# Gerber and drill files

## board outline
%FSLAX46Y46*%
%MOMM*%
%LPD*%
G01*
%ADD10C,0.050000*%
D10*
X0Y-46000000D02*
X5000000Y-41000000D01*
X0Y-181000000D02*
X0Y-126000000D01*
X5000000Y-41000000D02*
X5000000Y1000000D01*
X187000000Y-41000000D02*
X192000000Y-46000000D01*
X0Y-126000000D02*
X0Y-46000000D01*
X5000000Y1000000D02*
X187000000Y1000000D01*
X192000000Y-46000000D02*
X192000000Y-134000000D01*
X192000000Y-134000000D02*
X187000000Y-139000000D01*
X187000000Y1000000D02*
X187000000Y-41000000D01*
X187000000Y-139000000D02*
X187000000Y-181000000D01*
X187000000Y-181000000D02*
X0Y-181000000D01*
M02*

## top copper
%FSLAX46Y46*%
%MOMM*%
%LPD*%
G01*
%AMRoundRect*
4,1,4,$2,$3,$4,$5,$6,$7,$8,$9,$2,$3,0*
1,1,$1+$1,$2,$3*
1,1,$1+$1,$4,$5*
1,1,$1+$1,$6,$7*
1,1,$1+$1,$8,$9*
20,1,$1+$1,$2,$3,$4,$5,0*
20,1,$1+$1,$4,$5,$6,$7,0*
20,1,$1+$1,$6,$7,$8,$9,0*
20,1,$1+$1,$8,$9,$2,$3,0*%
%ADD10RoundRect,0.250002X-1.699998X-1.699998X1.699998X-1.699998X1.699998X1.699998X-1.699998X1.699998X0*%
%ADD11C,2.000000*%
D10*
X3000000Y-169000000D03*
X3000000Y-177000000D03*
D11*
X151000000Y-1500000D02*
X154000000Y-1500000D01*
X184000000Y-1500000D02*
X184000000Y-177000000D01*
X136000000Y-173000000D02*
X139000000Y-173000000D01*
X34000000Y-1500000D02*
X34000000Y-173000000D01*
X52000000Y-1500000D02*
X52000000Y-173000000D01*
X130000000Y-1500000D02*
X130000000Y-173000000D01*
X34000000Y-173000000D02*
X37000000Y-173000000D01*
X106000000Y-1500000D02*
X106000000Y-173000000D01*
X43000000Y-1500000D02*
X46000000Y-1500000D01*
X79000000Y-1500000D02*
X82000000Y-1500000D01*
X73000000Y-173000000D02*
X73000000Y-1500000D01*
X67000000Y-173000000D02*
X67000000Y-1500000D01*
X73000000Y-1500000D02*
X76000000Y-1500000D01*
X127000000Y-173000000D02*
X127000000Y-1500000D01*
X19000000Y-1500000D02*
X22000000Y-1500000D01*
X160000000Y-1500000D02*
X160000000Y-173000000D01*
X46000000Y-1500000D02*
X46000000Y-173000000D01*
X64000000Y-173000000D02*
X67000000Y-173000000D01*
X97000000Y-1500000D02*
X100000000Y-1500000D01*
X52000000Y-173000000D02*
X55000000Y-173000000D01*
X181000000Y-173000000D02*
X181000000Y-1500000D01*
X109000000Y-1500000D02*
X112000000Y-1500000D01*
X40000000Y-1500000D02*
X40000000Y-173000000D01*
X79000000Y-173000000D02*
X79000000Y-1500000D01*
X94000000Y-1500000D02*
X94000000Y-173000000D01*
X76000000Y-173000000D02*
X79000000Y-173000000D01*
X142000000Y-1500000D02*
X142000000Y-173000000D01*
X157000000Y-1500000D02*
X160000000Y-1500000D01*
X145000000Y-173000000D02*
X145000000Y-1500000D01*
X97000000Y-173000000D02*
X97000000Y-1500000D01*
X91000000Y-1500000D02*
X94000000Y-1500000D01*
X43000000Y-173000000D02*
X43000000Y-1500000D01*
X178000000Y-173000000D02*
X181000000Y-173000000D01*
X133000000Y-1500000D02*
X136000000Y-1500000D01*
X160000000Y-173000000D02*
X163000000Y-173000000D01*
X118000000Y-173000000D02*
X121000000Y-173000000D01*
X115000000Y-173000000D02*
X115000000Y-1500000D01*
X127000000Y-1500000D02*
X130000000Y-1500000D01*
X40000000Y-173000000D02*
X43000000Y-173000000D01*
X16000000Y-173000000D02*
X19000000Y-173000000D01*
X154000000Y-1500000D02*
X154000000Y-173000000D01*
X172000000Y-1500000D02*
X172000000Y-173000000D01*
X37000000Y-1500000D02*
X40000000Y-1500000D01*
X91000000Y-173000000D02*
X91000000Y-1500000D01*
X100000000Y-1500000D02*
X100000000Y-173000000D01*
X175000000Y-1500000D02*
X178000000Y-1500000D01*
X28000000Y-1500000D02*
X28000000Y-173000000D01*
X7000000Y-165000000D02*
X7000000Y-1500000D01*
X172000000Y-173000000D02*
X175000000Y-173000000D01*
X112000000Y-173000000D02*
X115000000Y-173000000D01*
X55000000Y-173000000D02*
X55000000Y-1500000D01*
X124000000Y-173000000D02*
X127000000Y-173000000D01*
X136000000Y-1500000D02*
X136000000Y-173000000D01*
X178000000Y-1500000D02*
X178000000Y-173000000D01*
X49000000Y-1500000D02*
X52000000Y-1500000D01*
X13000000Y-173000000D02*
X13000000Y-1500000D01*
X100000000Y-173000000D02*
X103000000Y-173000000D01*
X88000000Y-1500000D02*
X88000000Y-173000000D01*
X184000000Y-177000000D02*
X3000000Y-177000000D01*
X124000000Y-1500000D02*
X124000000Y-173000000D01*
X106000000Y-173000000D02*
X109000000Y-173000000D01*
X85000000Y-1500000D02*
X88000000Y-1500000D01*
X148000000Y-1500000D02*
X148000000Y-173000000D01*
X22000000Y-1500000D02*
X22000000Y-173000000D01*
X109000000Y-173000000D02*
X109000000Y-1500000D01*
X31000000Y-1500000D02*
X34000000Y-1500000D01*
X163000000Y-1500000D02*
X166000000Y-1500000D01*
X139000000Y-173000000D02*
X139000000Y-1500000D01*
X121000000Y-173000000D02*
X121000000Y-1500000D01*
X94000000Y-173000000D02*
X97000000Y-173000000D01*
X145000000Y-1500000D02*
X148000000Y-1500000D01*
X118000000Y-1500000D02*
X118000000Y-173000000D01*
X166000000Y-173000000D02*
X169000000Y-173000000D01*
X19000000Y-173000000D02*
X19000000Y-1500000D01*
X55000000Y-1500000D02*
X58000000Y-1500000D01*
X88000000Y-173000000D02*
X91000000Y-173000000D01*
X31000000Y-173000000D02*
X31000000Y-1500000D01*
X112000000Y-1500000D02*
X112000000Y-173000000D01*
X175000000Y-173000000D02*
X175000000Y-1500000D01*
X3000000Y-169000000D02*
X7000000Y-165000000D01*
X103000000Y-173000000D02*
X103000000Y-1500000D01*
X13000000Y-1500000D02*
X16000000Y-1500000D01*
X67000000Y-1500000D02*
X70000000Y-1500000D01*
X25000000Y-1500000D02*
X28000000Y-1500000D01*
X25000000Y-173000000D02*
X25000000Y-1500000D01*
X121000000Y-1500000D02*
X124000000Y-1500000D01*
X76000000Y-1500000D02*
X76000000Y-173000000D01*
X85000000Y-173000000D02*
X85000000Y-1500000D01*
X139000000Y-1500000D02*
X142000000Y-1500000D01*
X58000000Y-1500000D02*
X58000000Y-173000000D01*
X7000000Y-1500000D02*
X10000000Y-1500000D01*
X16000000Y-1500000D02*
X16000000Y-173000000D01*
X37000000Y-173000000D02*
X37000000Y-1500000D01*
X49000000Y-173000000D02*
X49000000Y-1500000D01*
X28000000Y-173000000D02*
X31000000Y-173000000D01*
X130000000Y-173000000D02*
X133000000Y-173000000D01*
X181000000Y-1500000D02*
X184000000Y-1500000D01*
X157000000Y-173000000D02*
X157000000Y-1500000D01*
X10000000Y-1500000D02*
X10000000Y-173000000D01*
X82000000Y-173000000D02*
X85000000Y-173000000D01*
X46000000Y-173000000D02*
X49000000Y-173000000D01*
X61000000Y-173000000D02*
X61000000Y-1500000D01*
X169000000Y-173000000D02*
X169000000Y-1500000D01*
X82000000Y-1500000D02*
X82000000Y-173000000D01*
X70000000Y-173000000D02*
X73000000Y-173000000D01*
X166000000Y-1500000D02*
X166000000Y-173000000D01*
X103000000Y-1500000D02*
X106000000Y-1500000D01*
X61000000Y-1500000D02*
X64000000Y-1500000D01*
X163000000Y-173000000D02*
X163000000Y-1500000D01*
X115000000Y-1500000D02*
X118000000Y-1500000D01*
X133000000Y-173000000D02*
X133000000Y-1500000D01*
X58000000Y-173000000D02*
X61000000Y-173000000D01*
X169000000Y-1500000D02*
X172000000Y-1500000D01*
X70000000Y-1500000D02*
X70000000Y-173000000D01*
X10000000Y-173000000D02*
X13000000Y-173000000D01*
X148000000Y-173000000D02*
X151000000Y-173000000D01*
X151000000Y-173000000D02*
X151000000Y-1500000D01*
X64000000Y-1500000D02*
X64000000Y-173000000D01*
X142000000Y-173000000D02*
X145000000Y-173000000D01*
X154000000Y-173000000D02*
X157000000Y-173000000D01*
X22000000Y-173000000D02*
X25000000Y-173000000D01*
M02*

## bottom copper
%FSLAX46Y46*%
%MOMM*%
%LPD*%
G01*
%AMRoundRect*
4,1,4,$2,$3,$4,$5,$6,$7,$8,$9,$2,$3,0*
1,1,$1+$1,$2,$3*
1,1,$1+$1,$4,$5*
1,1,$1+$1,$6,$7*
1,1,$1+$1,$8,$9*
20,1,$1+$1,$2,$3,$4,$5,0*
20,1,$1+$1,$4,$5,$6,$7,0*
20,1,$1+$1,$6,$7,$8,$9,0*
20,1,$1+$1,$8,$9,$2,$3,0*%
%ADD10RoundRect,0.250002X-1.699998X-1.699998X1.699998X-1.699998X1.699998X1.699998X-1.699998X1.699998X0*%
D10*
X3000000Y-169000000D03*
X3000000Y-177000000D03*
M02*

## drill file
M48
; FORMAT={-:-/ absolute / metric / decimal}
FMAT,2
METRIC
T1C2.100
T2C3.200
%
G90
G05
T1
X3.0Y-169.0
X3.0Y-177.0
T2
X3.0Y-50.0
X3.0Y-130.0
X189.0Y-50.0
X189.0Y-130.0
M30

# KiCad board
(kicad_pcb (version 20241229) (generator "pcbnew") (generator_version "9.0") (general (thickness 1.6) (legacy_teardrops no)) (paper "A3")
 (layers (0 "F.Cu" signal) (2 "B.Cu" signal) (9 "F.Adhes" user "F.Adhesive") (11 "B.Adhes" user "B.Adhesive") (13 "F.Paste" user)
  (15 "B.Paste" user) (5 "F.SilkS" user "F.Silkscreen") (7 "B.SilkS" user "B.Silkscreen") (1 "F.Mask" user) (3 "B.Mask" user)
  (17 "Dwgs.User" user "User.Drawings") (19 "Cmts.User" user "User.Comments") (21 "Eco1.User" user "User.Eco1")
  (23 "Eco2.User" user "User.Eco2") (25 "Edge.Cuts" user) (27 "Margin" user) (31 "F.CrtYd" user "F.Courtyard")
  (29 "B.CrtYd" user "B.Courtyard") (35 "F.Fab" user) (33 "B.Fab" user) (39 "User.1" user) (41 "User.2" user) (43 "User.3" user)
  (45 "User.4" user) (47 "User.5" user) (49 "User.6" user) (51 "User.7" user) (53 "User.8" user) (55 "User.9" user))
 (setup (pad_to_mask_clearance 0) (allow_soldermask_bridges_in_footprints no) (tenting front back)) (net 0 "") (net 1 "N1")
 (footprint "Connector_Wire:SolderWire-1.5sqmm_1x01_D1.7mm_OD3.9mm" (layer "F.Cu") (at 3 169)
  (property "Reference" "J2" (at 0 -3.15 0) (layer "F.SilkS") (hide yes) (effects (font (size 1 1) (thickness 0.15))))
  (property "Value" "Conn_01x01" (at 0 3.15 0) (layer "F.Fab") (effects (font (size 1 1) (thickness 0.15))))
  (pad "1" thru_hole roundrect (at 0 0) (size 3.9 3.9) (drill 2.1) (layers "*.Cu" "*.Mask") (remove_unused_layers no)
   (roundrect_rratio 0.064103) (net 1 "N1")))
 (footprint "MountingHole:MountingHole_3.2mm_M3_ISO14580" (layer "F.Cu") (at 189 50)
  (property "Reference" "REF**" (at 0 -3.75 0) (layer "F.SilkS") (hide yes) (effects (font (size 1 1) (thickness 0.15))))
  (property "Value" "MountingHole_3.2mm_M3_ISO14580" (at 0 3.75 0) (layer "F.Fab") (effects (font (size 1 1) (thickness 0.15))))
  (pad "" np_thru_hole circle (at 0 0) (size 3.2 3.2) (drill 3.2) (layers "*.Cu" "*.Mask")))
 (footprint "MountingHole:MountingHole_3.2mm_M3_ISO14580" (layer "F.Cu") (at 3 130)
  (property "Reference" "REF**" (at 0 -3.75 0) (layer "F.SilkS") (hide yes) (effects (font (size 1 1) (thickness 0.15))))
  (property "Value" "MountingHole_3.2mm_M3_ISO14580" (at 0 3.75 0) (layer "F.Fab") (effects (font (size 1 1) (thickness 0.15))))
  (pad "" np_thru_hole circle (at 0 0) (size 3.2 3.2) (drill 3.2) (layers "*.Cu" "*.Mask")))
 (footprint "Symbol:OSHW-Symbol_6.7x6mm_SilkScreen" (layer "F.Cu") (at 12 175)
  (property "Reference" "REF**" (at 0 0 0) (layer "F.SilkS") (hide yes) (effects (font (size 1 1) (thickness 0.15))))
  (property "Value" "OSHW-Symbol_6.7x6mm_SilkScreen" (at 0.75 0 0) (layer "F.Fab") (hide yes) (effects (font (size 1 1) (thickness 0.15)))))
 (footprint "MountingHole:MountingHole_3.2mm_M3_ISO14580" (layer "F.Cu") (at 189 130)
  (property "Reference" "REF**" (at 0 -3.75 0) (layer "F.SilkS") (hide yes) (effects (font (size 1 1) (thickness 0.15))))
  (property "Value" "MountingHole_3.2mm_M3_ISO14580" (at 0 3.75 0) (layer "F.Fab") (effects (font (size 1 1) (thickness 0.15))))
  (pad "" np_thru_hole circle (at 0 0) (size 3.2 3.2) (drill 3.2) (layers "*.Cu" "*.Mask")))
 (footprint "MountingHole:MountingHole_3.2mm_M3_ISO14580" (layer "F.Cu") (at 3 50)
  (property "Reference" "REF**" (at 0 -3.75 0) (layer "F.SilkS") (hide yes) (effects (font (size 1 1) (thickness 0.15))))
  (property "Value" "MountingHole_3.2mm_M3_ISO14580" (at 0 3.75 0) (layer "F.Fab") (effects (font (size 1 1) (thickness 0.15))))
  (pad "" np_thru_hole circle (at 0 0) (size 3.2 3.2) (drill 3.2) (layers "*.Cu" "*.Mask")))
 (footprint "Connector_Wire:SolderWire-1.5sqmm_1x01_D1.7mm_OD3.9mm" (layer "F.Cu") (at 3 177)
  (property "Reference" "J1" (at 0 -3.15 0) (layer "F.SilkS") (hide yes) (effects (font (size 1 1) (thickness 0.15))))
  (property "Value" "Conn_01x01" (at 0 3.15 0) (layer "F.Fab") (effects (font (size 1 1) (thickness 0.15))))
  (pad "1" thru_hole roundrect (at 0 0) (size 3.9 3.9) (drill 2.1) (layers "*.Cu" "*.Mask") (remove_unused_layers no)
   (roundrect_rratio 0.064103) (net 1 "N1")))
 (gr_line (start 0 46) (end 5 41) (stroke (width 0.05) (type default)) (layer "Edge.Cuts"))
 (gr_line (start 0 181) (end 0 126) (stroke (width 0.05) (type default)) (layer "Edge.Cuts"))
 (gr_line (start 5 41) (end 5 -1) (stroke (width 0.05) (type default)) (layer "Edge.Cuts"))
 (gr_line (start 187 41) (end 192 46) (stroke (width 0.05) (type default)) (layer "Edge.Cuts"))
 (gr_line (start 0 126) (end 0 46) (stroke (width 0.05) (type default)) (layer "Edge.Cuts"))
 (gr_line (start 5 -1) (end 187 -1) (stroke (width 0.05) (type default)) (layer "Edge.Cuts"))
 (gr_line (start 192 46) (end 192 134) (stroke (width 0.05) (type default)) (layer "Edge.Cuts"))
 (gr_line (start 192 134) (end 187 139) (stroke (width 0.05) (type default)) (layer "Edge.Cuts"))
 (gr_line (start 187 -1) (end 187 41) (stroke (width 0.05) (type default)) (layer "Edge.Cuts"))
 (gr_line (start 187 139) (end 187 181) (stroke (width 0.05) (type default)) (layer "Edge.Cuts"))
 (gr_line (start 187 181) (end 0 181) (stroke (width 0.05) (type default)) (layer "Edge.Cuts"))
 (segment (start 151 1.5) (end 154 1.5) (width 2) (layer "F.Cu") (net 1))
 (segment (start 184 1.5) (end 184 177) (width 2) (layer "F.Cu") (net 1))
 (segment (start 136 173) (end 139 173) (width 2) (layer "F.Cu") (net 1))
 (segment (start 34 1.5) (end 34 173) (width 2) (layer "F.Cu") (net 1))
 (segment (start 52 1.5) (end 52 173) (width 2) (layer "F.Cu") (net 1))
 (segment (start 130 1.5) (end 130 173) (width 2) (layer "F.Cu") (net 1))
 (segment (start 34 173) (end 37 173) (width 2) (layer "F.Cu") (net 1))
 (segment (start 106 1.5) (end 106 173) (width 2) (layer "F.Cu") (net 1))
 (segment (start 43 1.5) (end 46 1.5) (width 2) (layer "F.Cu") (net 1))
 (segment (start 79 1.5) (end 82 1.5) (width 2) (layer "F.Cu") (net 1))
 (segment (start 73 173) (end 73 1.5) (width 2) (layer "F.Cu") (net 1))
 (segment (start 67 173) (end 67 1.5) (width 2) (layer "F.Cu") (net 1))
 (segment (start 73 1.5) (end 76 1.5) (width 2) (layer "F.Cu") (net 1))
 (segment (start 127 173) (end 127 1.5) (width 2) (layer "F.Cu") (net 1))
 (segment (start 19 1.5) (end 22 1.5) (width 2) (layer "F.Cu") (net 1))
 (segment (start 160 1.5) (end 160 173) (width 2) (layer "F.Cu") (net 1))
 (segment (start 46 1.5) (end 46 173) (width 2) (layer "F.Cu") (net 1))
 (segment (start 64 173) (end 67 173) (width 2) (layer "F.Cu") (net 1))
 (segment (start 97 1.5) (end 100 1.5) (width 2) (layer "F.Cu") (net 1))
 (segment (start 52 173) (end 55 173) (width 2) (layer "F.Cu") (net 1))
 (segment (start 181 173) (end 181 1.5) (width 2) (layer "F.Cu") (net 1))
 (segment (start 109 1.5) (end 112 1.5) (width 2) (layer "F.Cu") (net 1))
 (segment (start 40 1.5) (end 40 173) (width 2) (layer "F.Cu") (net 1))
 (segment (start 79 173) (end 79 1.5) (width 2) (layer "F.Cu") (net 1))
 (segment (start 94 1.5) (end 94 173) (width 2) (layer "F.Cu") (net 1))
 (segment (start 76 173) (end 79 173) (width 2) (layer "F.Cu") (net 1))
 (segment (start 142 1.5) (end 142 173) (width 2) (layer "F.Cu") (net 1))
 (segment (start 157 1.5) (end 160 1.5) (width 2) (layer "F.Cu") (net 1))
 (segment (start 145 173) (end 145 1.5) (width 2) (layer "F.Cu") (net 1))
 (segment (start 97 173) (end 97 1.5) (width 2) (layer "F.Cu") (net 1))
 (segment (start 91 1.5) (end 94 1.5) (width 2) (layer "F.Cu") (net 1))
 (segment (start 43 173) (end 43 1.5) (width 2) (layer "F.Cu") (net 1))
 (segment (start 178 173) (end 181 173) (width 2) (layer "F.Cu") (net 1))
 (segment (start 133 1.5) (end 136 1.5) (width 2) (layer "F.Cu") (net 1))
 (segment (start 160 173) (end 163 173) (width 2) (layer "F.Cu") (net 1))
 (segment (start 118 173) (end 121 173) (width 2) (layer "F.Cu") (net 1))
 (segment (start 115 173) (end 115 1.5) (width 2) (layer "F.Cu") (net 1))
 (segment (start 127 1.5) (end 130 1.5) (width 2) (layer "F.Cu") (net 1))
 (segment (start 40 173) (end 43 173) (width 2) (layer "F.Cu") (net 1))
 (segment (start 16 173) (end 19 173) (width 2) (layer "F.Cu") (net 1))
 (segment (start 154 1.5) (end 154 173) (width 2) (layer "F.Cu") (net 1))
 (segment (start 172 1.5) (end 172 173) (width 2) (layer "F.Cu") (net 1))
 (segment (start 37 1.5) (end 40 1.5) (width 2) (layer "F.Cu") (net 1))
 (segment (start 91 173) (end 91 1.5) (width 2) (layer "F.Cu") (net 1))
 (segment (start 100 1.5) (end 100 173) (width 2) (layer "F.Cu") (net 1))
 (segment (start 175 1.5) (end 178 1.5) (width 2) (layer "F.Cu") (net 1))
 (segment (start 28 1.5) (end 28 173) (width 2) (layer "F.Cu") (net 1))
 (segment (start 7 165) (end 7 1.5) (width 2) (layer "F.Cu") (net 1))
 (segment (start 172 173) (end 175 173) (width 2) (layer "F.Cu") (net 1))
 (segment (start 112 173) (end 115 173) (width 2) (layer "F.Cu") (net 1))
 (segment (start 55 173) (end 55 1.5) (width 2) (layer "F.Cu") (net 1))
 (segment (start 124 173) (end 127 173) (width 2) (layer "F.Cu") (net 1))
 (segment (start 136 1.5) (end 136 173) (width 2) (layer "F.Cu") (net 1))
 (segment (start 178 1.5) (end 178 173) (width 2) (layer "F.Cu") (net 1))
 (segment (start 49 1.5) (end 52 1.5) (width 2) (layer "F.Cu") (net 1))
 (segment (start 13 173) (end 13 1.5) (width 2) (layer "F.Cu") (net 1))
 (segment (start 100 173) (end 103 173) (width 2) (layer "F.Cu") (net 1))
 (segment (start 88 1.5) (end 88 173) (width 2) (layer "F.Cu") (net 1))
 (segment (start 184 177) (end 3 177) (width 2) (layer "F.Cu") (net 1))
 (segment (start 124 1.5) (end 124 173) (width 2) (layer "F.Cu") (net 1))
 (segment (start 106 173) (end 109 173) (width 2) (layer "F.Cu") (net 1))
 (segment (start 85 1.5) (end 88 1.5) (width 2) (layer "F.Cu") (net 1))
 (segment (start 148 1.5) (end 148 173) (width 2) (layer "F.Cu") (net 1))
 (segment (start 22 1.5) (end 22 173) (width 2) (layer "F.Cu") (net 1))
 (segment (start 109 173) (end 109 1.5) (width 2) (layer "F.Cu") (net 1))
 (segment (start 31 1.5) (end 34 1.5) (width 2) (layer "F.Cu") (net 1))
 (segment (start 163 1.5) (end 166 1.5) (width 2) (layer "F.Cu") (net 1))
 (segment (start 139 173) (end 139 1.5) (width 2) (layer "F.Cu") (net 1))
 (segment (start 121 173) (end 121 1.5) (width 2) (layer "F.Cu") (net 1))
 (segment (start 94 173) (end 97 173) (width 2) (layer "F.Cu") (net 1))
 (segment (start 145 1.5) (end 148 1.5) (width 2) (layer "F.Cu") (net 1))
 (segment (start 118 1.5) (end 118 173) (width 2) (layer "F.Cu") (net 1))
 (segment (start 166 173) (end 169 173) (width 2) (layer "F.Cu") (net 1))
 (segment (start 19 173) (end 19 1.5) (width 2) (layer "F.Cu") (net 1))
 (segment (start 55 1.5) (end 58 1.5) (width 2) (layer "F.Cu") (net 1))
 (segment (start 88 173) (end 91 173) (width 2) (layer "F.Cu") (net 1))
 (segment (start 31 173) (end 31 1.5) (width 2) (layer "F.Cu") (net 1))
 (segment (start 112 1.5) (end 112 173) (width 2) (layer "F.Cu") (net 1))
 (segment (start 175 173) (end 175 1.5) (width 2) (layer "F.Cu") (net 1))
 (segment (start 3 169) (end 7 165) (width 2) (layer "F.Cu") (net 1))
 (segment (start 103 173) (end 103 1.5) (width 2) (layer "F.Cu") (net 1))
 (segment (start 13 1.5) (end 16 1.5) (width 2) (layer "F.Cu") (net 1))
 (segment (start 67 1.5) (end 70 1.5) (width 2) (layer "F.Cu") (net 1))
 (segment (start 25 1.5) (end 28 1.5) (width 2) (layer "F.Cu") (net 1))
 (segment (start 25 173) (end 25 1.5) (width 2) (layer "F.Cu") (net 1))
 (segment (start 121 1.5) (end 124 1.5) (width 2) (layer "F.Cu") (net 1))
 (segment (start 76 1.5) (end 76 173) (width 2) (layer "F.Cu") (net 1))
 (segment (start 85 173) (end 85 1.5) (width 2) (layer "F.Cu") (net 1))
 (segment (start 139 1.5) (end 142 1.5) (width 2) (layer "F.Cu") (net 1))
 (segment (start 58 1.5) (end 58 173) (width 2) (layer "F.Cu") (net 1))
 (segment (start 7 1.5) (end 10 1.5) (width 2) (layer "F.Cu") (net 1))
 (segment (start 16 1.5) (end 16 173) (width 2) (layer "F.Cu") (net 1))
 (segment (start 37 173) (end 37 1.5) (width 2) (layer "F.Cu") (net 1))
 (segment (start 49 173) (end 49 1.5) (width 2) (layer "F.Cu") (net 1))
 (segment (start 28 173) (end 31 173) (width 2) (layer "F.Cu") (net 1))
 (segment (start 130 173) (end 133 173) (width 2) (layer "F.Cu") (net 1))
 (segment (start 181 1.5) (end 184 1.5) (width 2) (layer "F.Cu") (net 1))
 (segment (start 157 173) (end 157 1.5) (width 2) (layer "F.Cu") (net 1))
 (segment (start 10 1.5) (end 10 173) (width 2) (layer "F.Cu") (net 1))
 (segment (start 82 173) (end 85 173) (width 2) (layer "F.Cu") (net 1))
 (segment (start 46 173) (end 49 173) (width 2) (layer "F.Cu") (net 1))
 (segment (start 61 173) (end 61 1.5) (width 2) (layer "F.Cu") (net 1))
 (segment (start 169 173) (end 169 1.5) (width 2) (layer "F.Cu") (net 1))
 (segment (start 82 1.5) (end 82 173) (width 2) (layer "F.Cu") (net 1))
 (segment (start 70 173) (end 73 173) (width 2) (layer "F.Cu") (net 1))
 (segment (start 166 1.5) (end 166 173) (width 2) (layer "F.Cu") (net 1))
 (segment (start 103 1.5) (end 106 1.5) (width 2) (layer "F.Cu") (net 1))
 (segment (start 61 1.5) (end 64 1.5) (width 2) (layer "F.Cu") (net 1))
 (segment (start 163 173) (end 163 1.5) (width 2) (layer "F.Cu") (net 1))
 (segment (start 115 1.5) (end 118 1.5) (width 2) (layer "F.Cu") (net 1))
 (segment (start 133 173) (end 133 1.5) (width 2) (layer "F.Cu") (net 1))
 (segment (start 58 173) (end 61 173) (width 2) (layer "F.Cu") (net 1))
 (segment (start 169 1.5) (end 172 1.5) (width 2) (layer "F.Cu") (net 1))
 (segment (start 70 1.5) (end 70 173) (width 2) (layer "F.Cu") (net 1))
 (segment (start 10 173) (end 13 173) (width 2) (layer "F.Cu") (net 1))
 (segment (start 148 173) (end 151 173) (width 2) (layer "F.Cu") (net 1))
 (segment (start 151 173) (end 151 1.5) (width 2) (layer "F.Cu") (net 1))
 (segment (start 64 1.5) (end 64 173) (width 2) (layer "F.Cu") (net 1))
 (segment (start 142 173) (end 145 173) (width 2) (layer "F.Cu") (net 1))
 (segment (start 154 173) (end 157 173) (width 2) (layer "F.Cu") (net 1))
 (segment (start 22 173) (end 25 173) (width 2) (layer "F.Cu") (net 1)))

